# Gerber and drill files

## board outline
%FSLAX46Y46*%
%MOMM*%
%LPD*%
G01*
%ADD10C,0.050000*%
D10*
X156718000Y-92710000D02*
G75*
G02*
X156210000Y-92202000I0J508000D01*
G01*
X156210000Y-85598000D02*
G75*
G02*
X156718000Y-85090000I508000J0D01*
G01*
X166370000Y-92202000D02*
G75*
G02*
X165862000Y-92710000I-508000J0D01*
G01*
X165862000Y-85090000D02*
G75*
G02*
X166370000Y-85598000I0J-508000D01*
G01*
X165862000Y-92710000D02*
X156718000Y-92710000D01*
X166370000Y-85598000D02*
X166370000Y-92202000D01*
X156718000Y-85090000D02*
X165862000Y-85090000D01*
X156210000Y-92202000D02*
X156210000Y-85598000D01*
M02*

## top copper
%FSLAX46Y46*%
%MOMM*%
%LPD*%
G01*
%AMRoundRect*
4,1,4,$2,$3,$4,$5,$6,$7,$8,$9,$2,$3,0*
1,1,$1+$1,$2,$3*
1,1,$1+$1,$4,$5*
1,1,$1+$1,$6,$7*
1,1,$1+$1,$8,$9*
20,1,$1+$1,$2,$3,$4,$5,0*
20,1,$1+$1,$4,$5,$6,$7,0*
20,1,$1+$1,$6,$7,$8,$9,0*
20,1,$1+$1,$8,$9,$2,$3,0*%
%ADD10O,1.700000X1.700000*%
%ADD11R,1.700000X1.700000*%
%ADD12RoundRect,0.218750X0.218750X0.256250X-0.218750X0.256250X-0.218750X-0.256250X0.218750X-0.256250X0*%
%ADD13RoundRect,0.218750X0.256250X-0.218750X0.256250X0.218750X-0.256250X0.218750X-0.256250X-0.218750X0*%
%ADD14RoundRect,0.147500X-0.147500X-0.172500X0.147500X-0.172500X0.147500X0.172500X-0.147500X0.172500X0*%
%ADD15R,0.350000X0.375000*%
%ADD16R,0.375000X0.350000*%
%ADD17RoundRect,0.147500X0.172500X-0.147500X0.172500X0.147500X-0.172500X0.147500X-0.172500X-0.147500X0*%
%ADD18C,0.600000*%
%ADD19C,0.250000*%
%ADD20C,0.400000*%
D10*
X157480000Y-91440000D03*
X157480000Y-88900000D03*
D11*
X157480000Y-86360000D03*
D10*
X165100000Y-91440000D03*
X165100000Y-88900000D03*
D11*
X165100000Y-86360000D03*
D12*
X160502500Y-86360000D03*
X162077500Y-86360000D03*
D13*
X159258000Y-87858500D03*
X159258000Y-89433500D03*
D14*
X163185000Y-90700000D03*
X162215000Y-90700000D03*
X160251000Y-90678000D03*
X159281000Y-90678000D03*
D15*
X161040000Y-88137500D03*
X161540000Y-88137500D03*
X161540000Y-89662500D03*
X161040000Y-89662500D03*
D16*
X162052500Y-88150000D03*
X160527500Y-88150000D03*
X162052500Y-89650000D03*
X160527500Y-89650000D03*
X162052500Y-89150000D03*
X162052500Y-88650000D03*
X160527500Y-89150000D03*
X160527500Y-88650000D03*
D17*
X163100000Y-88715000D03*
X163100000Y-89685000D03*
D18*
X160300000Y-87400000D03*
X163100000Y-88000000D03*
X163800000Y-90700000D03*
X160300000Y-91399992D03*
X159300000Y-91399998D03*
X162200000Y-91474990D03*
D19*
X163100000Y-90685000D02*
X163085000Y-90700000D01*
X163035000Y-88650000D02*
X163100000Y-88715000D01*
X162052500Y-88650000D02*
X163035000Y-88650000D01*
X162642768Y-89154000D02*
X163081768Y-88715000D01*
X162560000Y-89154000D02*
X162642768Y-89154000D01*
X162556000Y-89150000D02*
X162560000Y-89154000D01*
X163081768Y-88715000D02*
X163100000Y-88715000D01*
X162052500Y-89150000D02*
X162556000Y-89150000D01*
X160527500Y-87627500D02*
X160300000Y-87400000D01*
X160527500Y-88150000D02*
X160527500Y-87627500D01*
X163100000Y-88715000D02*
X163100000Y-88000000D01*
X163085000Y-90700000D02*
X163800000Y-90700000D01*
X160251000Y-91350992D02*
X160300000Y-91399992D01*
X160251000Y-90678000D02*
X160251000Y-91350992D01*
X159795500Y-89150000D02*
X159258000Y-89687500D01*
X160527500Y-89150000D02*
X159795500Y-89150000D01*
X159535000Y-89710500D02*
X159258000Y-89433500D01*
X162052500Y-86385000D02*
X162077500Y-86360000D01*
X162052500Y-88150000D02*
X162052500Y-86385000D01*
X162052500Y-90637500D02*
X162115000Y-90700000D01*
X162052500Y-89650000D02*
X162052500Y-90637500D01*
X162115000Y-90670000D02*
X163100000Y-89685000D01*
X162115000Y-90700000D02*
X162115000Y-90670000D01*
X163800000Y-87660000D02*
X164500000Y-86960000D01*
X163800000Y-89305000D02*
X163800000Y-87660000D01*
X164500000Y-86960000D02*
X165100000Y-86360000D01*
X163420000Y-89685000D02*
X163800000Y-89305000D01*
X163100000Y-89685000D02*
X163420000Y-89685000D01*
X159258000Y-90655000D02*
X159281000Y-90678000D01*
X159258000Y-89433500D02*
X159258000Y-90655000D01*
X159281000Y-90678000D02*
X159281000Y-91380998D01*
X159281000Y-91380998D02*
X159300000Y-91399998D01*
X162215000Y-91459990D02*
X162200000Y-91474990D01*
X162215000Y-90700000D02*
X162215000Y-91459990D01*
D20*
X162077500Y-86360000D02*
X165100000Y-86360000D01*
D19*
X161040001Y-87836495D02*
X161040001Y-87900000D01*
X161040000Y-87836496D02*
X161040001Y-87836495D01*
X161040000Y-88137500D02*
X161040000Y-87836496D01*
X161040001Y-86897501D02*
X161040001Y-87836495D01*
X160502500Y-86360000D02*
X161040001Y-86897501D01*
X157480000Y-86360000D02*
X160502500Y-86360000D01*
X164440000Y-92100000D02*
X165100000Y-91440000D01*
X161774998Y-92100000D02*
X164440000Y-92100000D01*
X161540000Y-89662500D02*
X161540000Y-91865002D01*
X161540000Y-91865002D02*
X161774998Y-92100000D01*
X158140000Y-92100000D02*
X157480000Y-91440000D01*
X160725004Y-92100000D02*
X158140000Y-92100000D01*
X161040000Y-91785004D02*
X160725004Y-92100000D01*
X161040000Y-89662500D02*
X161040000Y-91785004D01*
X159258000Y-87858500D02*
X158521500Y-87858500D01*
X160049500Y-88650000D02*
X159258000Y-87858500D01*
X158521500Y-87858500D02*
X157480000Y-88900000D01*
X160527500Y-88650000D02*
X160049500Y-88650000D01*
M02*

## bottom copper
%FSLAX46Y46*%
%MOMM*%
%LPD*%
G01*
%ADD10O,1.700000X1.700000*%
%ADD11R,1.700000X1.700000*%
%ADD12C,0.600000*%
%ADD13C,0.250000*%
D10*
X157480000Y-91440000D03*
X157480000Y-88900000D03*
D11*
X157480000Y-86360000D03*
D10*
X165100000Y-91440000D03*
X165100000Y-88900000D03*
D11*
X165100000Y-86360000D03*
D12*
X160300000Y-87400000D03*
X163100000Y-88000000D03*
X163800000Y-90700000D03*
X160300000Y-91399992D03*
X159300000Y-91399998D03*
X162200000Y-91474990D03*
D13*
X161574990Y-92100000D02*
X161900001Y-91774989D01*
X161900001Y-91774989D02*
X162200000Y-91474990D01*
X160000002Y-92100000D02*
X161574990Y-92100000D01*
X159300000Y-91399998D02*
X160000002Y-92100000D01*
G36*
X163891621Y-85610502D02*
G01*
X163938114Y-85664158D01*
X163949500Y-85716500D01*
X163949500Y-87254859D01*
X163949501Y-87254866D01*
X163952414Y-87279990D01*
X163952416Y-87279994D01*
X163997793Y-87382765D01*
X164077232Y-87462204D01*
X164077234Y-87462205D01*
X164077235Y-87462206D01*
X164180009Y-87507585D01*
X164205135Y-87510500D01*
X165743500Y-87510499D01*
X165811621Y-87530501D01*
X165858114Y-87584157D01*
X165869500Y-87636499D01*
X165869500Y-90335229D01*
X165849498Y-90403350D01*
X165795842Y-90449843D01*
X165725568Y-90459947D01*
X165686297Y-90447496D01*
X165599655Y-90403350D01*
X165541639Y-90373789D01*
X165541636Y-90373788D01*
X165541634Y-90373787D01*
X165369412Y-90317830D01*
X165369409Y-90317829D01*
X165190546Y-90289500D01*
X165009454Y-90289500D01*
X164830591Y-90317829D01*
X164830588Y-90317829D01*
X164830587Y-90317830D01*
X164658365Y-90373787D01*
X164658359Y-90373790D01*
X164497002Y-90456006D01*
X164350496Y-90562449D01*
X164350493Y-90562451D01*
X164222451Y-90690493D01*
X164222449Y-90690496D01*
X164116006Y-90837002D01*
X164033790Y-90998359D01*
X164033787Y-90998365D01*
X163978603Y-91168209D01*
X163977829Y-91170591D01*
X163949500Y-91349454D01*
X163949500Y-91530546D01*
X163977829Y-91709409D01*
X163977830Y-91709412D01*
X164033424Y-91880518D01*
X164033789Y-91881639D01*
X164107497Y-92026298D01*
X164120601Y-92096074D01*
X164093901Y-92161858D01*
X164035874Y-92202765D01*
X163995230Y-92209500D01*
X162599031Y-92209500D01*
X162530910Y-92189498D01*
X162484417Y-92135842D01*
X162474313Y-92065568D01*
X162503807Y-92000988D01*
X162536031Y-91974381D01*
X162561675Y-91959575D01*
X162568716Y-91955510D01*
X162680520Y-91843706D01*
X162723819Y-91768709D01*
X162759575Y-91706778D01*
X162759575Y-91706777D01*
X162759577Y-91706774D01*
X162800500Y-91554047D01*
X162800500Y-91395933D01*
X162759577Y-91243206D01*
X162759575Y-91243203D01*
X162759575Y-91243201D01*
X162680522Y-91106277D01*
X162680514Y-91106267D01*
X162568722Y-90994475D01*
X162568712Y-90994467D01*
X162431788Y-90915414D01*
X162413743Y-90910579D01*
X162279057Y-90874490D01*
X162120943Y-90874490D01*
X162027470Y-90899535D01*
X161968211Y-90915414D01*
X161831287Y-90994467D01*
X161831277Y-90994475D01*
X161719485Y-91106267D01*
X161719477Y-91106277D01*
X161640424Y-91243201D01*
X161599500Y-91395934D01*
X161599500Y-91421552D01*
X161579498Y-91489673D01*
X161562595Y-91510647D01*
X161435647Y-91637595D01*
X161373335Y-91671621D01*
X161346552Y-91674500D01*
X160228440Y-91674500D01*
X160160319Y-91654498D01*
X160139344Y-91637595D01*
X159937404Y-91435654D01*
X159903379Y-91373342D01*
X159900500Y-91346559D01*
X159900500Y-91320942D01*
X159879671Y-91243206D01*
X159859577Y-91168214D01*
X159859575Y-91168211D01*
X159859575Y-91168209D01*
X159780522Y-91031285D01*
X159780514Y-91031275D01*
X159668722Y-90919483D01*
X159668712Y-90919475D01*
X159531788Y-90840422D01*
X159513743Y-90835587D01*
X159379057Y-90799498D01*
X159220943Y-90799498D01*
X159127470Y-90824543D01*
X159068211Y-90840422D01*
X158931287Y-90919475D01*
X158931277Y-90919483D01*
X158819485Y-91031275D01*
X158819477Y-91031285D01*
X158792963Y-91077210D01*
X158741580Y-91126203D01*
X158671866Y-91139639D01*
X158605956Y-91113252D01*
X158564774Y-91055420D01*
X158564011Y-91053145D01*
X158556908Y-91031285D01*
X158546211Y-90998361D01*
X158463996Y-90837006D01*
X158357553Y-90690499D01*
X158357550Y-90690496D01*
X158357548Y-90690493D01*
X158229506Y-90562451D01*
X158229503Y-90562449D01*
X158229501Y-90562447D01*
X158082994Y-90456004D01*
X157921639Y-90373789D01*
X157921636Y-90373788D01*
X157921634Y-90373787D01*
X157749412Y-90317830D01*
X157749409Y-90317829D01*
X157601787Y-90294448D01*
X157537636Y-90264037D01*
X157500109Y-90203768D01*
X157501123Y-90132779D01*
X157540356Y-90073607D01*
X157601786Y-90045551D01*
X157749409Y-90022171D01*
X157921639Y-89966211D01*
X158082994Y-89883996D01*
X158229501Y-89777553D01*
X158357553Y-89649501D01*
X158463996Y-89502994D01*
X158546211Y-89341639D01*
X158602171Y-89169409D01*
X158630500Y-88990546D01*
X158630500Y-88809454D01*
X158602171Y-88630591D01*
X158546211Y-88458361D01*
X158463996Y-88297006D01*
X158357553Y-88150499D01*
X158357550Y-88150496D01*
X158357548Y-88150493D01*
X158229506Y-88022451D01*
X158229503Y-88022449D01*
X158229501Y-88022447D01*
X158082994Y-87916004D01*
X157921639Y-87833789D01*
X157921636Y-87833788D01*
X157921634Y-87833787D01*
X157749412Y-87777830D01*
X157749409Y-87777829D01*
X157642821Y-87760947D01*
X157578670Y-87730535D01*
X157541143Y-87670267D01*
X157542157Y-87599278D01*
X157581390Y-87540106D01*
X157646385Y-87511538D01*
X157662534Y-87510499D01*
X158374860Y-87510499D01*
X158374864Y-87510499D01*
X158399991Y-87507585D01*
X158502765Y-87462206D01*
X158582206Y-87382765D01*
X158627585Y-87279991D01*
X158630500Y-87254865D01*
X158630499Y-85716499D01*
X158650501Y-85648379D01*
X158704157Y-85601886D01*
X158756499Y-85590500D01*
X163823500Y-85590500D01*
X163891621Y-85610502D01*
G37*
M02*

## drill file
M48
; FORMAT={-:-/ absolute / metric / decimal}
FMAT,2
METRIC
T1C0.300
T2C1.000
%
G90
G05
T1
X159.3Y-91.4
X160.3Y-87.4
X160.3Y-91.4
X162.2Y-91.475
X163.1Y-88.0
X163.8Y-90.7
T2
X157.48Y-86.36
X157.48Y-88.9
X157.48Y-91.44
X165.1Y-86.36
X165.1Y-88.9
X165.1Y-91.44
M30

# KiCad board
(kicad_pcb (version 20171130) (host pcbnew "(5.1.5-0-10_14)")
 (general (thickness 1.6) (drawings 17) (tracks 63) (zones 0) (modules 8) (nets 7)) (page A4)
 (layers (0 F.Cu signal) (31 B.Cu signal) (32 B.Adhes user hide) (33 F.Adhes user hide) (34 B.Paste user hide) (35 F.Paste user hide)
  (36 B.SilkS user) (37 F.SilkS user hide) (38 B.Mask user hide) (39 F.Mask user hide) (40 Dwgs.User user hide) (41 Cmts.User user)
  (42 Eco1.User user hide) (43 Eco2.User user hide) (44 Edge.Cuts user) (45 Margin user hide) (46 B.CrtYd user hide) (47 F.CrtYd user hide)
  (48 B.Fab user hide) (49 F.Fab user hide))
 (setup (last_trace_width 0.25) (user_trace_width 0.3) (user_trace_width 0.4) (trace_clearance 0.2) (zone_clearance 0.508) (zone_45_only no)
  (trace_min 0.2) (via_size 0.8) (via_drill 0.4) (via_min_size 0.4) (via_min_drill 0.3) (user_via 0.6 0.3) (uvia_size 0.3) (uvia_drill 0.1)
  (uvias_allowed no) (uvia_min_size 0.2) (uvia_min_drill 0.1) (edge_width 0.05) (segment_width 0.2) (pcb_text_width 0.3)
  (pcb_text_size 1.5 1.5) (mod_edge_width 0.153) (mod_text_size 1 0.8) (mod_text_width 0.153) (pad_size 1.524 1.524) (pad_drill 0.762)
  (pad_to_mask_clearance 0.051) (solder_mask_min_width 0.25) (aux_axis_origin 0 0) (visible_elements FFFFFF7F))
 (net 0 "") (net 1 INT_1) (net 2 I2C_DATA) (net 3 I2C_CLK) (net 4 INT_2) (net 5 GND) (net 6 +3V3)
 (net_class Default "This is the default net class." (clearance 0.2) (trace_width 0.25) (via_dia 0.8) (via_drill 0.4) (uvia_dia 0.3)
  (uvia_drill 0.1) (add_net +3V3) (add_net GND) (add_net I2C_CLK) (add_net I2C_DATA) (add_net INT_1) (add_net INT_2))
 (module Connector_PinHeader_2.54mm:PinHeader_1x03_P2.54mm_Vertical (layer B.Cu) (at 157.48 86.36 180)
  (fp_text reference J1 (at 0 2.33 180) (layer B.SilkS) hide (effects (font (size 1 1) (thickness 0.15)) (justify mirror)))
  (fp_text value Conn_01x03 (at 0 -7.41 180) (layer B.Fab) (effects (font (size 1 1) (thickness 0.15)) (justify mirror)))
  (pad 3 thru_hole oval (at 0 -5.08 180) (size 1.7 1.7) (drill 1) (layers *.Cu *.Mask) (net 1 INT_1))
  (pad 2 thru_hole oval (at 0 -2.54 180) (size 1.7 1.7) (drill 1) (layers *.Cu *.Mask) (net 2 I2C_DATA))
  (pad 1 thru_hole rect (at 0 0 180) (size 1.7 1.7) (drill 1) (layers *.Cu *.Mask) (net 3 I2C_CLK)))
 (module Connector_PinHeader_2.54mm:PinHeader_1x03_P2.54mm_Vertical (layer B.Cu) (at 165.1 86.36 180)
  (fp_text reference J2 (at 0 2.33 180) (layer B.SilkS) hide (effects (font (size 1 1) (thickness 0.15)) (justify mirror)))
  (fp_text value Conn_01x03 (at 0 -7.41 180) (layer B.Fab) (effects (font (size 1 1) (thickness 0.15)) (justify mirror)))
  (pad 3 thru_hole oval (at 0 -5.08 180) (size 1.7 1.7) (drill 1) (layers *.Cu *.Mask) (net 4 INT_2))
  (pad 2 thru_hole oval (at 0 -2.54 180) (size 1.7 1.7) (drill 1) (layers *.Cu *.Mask) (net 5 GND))
  (pad 1 thru_hole rect (at 0 0 180) (size 1.7 1.7) (drill 1) (layers *.Cu *.Mask) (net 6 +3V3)))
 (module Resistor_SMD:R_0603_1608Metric (layer F.Cu) (at 161.29 86.36 180)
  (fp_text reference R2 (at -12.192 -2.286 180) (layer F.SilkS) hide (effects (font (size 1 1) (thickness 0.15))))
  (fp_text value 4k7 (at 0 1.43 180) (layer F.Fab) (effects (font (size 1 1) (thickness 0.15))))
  (pad 2 smd roundrect (at 0.7875 0 180) (size 0.875 0.95) (layers F.Cu F.Paste F.Mask) (roundrect_rratio 0.25) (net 3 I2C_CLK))
  (pad 1 smd roundrect (at -0.7875 0 180) (size 0.875 0.95) (layers F.Cu F.Paste F.Mask) (roundrect_rratio 0.25) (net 6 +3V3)))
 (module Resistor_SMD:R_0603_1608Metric (layer F.Cu) (at 159.258 88.646 90)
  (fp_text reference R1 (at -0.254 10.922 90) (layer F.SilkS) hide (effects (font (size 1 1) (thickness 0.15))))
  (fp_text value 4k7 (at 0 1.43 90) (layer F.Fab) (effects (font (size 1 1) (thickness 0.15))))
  (pad 2 smd roundrect (at 0.7875 0 90) (size 0.875 0.95) (layers F.Cu F.Paste F.Mask) (roundrect_rratio 0.25) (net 2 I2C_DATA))
  (pad 1 smd roundrect (at -0.7875 0 90) (size 0.875 0.95) (layers F.Cu F.Paste F.Mask) (roundrect_rratio 0.25) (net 6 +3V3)))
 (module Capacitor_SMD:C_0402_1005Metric (layer F.Cu) (at 162.7 90.7)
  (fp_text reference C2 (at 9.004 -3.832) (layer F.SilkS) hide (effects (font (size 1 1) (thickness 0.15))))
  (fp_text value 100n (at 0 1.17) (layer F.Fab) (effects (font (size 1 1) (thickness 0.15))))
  (pad 2 smd roundrect (at 0.485 0) (size 0.59 0.64) (layers F.Cu F.Paste F.Mask) (roundrect_rratio 0.25) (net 5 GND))
  (pad 1 smd roundrect (at -0.485 0) (size 0.59 0.64) (layers F.Cu F.Paste F.Mask) (roundrect_rratio 0.25) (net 6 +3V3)))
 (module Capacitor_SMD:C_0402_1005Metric (layer F.Cu) (at 159.766 90.678)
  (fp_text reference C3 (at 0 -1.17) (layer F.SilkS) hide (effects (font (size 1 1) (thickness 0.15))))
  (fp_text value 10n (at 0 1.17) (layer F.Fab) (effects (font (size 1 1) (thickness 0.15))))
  (pad 2 smd roundrect (at 0.485 0) (size 0.59 0.64) (layers F.Cu F.Paste F.Mask) (roundrect_rratio 0.25) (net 5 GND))
  (pad 1 smd roundrect (at -0.485 0) (size 0.59 0.64) (layers F.Cu F.Paste F.Mask) (roundrect_rratio 0.25) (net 6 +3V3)))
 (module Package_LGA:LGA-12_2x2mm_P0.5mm (layer F.Cu) (at 161.29 88.9)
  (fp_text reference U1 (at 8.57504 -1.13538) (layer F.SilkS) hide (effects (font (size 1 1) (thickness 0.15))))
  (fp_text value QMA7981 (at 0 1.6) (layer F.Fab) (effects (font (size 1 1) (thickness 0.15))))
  (pad 12 smd rect (at -0.25 -0.7625 90) (size 0.375 0.35) (layers F.Cu F.Paste F.Mask) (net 3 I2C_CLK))
  (pad 11 smd rect (at 0.25 -0.7625 90) (size 0.375 0.35) (layers F.Cu F.Paste F.Mask))
  (pad 6 smd rect (at 0.25 0.7625 90) (size 0.375 0.35) (layers F.Cu F.Paste F.Mask) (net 4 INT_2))
  (pad 5 smd rect (at -0.25 0.7625 90) (size 0.375 0.35) (layers F.Cu F.Paste F.Mask) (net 1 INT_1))
  (pad 10 smd rect (at 0.7625 -0.75) (size 0.375 0.35) (layers F.Cu F.Paste F.Mask) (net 6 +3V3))
  (pad 1 smd rect (at -0.7625 -0.75) (size 0.375 0.35) (layers F.Cu F.Paste F.Mask) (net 5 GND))
  (pad 7 smd rect (at 0.7625 0.75) (size 0.375 0.35) (layers F.Cu F.Paste F.Mask) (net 6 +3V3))
  (pad 4 smd rect (at -0.7625 0.75) (size 0.375 0.35) (layers F.Cu F.Paste F.Mask))
  (pad 8 smd rect (at 0.7625 0.25) (size 0.375 0.35) (layers F.Cu F.Paste F.Mask) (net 5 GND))
  (pad 9 smd rect (at 0.7625 -0.25) (size 0.375 0.35) (layers F.Cu F.Paste F.Mask) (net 5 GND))
  (pad 3 smd rect (at -0.7625 0.25) (size 0.375 0.35) (layers F.Cu F.Paste F.Mask) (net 6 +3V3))
  (pad 2 smd rect (at -0.7625 -0.25) (size 0.375 0.35) (layers F.Cu F.Paste F.Mask) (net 2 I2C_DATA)))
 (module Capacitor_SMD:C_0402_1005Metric (layer F.Cu) (at 163.1 89.2 90)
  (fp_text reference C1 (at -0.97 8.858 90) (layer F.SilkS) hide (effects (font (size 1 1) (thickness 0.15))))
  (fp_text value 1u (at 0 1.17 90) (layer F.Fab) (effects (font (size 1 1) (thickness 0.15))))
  (pad 2 smd roundrect (at 0.485 0 90) (size 0.59 0.64) (layers F.Cu F.Paste F.Mask) (roundrect_rratio 0.25) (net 5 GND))
  (pad 1 smd roundrect (at -0.485 0 90) (size 0.59 0.64) (layers F.Cu F.Paste F.Mask) (roundrect_rratio 0.25) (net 6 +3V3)))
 (gr_arc (start 156.718 92.202) (end 156.21 92.202) (angle -90) (layer Edge.Cuts) (width 0.05))
 (gr_arc (start 156.718 85.598) (end 156.718 85.09) (angle -90) (layer Edge.Cuts) (width 0.05))
 (gr_arc (start 165.862 92.202) (end 165.862 92.71) (angle -90) (layer Edge.Cuts) (width 0.05))
 (gr_arc (start 165.862 85.598) (end 166.37 85.598) (angle -90) (layer Edge.Cuts) (width 0.05))
 (gr_line (start 165.862 92.71) (end 156.718 92.71) (layer Edge.Cuts) (width 0.05))
 (gr_line (start 166.37 85.598) (end 166.37 92.202) (layer Edge.Cuts) (width 0.05))
 (gr_line (start 156.718 85.09) (end 165.862 85.09) (layer Edge.Cuts) (width 0.05))
 (gr_line (start 156.21 92.202) (end 156.21 85.598) (layer Edge.Cuts) (width 0.05))
 (segment (start 163.1 90.685) (end 163.085 90.7) (width 0.25) (layer F.Cu) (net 5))
 (segment (start 163.035 88.65) (end 163.1 88.715) (width 0.25) (layer F.Cu) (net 5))
 (segment (start 162.0525 88.65) (end 163.035 88.65) (width 0.25) (layer F.Cu) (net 5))
 (segment (start 162.642768 89.154) (end 163.081768 88.715) (width 0.25) (layer F.Cu) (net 5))
 (segment (start 162.56 89.154) (end 162.642768 89.154) (width 0.25) (layer F.Cu) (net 5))
 (segment (start 162.556 89.15) (end 162.56 89.154) (width 0.25) (layer F.Cu) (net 5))
 (segment (start 163.081768 88.715) (end 163.1 88.715) (width 0.25) (layer F.Cu) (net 5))
 (segment (start 162.0525 89.15) (end 162.556 89.15) (width 0.25) (layer F.Cu) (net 5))
 (via (at 160.3 87.4) (size 0.6) (drill 0.3) (layers F.Cu B.Cu) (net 5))
 (segment (start 160.5275 87.6275) (end 160.3 87.4) (width 0.25) (layer F.Cu) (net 5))
 (segment (start 160.5275 88.15) (end 160.5275 87.6275) (width 0.25) (layer F.Cu) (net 5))
 (via (at 163.1 88) (size 0.6) (drill 0.3) (layers F.Cu B.Cu) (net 5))
 (segment (start 163.1 88.715) (end 163.1 88) (width 0.25) (layer F.Cu) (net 5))
 (segment (start 163.085 90.7) (end 163.8 90.7) (width 0.25) (layer F.Cu) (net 5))
 (via (at 163.8 90.7) (size 0.6) (drill 0.3) (layers F.Cu B.Cu) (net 5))
 (via (at 160.3 91.399992) (size 0.6) (drill 0.3) (layers F.Cu B.Cu) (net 5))
 (segment (start 160.251 91.350992) (end 160.3 91.399992) (width 0.25) (layer F.Cu) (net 5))
 (segment (start 160.251 90.678) (end 160.251 91.350992) (width 0.25) (layer F.Cu) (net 5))
 (segment (start 159.7955 89.15) (end 159.258 89.6875) (width 0.25) (layer F.Cu) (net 6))
 (segment (start 160.5275 89.15) (end 159.7955 89.15) (width 0.25) (layer F.Cu) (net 6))
 (segment (start 159.535 89.7105) (end 159.258 89.4335) (width 0.25) (layer F.Cu) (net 6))
 (segment (start 162.0525 86.385) (end 162.0775 86.36) (width 0.25) (layer F.Cu) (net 6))
 (segment (start 162.0525 88.15) (end 162.0525 86.385) (width 0.25) (layer F.Cu) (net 6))
 (segment (start 162.0525 90.6375) (end 162.115 90.7) (width 0.25) (layer F.Cu) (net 6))
 (segment (start 162.0525 89.65) (end 162.0525 90.6375) (width 0.25) (layer F.Cu) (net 6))
 (segment (start 162.115 90.67) (end 163.1 89.685) (width 0.25) (layer F.Cu) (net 6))
 (segment (start 162.115 90.7) (end 162.115 90.67) (width 0.25) (layer F.Cu) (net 6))
 (segment (start 163.8 87.66) (end 164.5 86.96) (width 0.25) (layer F.Cu) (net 6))
 (segment (start 163.8 89.305) (end 163.8 87.66) (width 0.25) (layer F.Cu) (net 6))
 (segment (start 164.5 86.96) (end 165.1 86.36) (width 0.25) (layer F.Cu) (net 6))
 (segment (start 163.42 89.685) (end 163.8 89.305) (width 0.25) (layer F.Cu) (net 6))
 (segment (start 163.1 89.685) (end 163.42 89.685) (width 0.25) (layer F.Cu) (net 6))
 (segment (start 159.258 90.655) (end 159.281 90.678) (width 0.25) (layer F.Cu) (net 6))
 (segment (start 159.258 89.4335) (end 159.258 90.655) (width 0.25) (layer F.Cu) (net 6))
 (via (at 159.3 91.399998) (size 0.6) (drill 0.3) (layers F.Cu B.Cu) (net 6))
 (segment (start 159.281 90.678) (end 159.281 91.380998) (width 0.25) (layer F.Cu) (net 6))
 (segment (start 159.281 91.380998) (end 159.3 91.399998) (width 0.25) (layer F.Cu) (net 6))
 (via (at 162.2 91.47499) (size 0.6) (drill 0.3) (layers F.Cu B.Cu) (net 6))
 (segment (start 161.57499 92.1) (end 161.900001 91.774989) (width 0.25) (layer B.Cu) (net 6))
 (segment (start 162.215 91.45999) (end 162.2 91.47499) (width 0.25) (layer F.Cu) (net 6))
 (segment (start 161.900001 91.774989) (end 162.2 91.47499) (width 0.25) (layer B.Cu) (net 6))
 (segment (start 160.000002 92.1) (end 161.57499 92.1) (width 0.25) (layer B.Cu) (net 6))
 (segment (start 162.215 90.7) (end 162.215 91.45999) (width 0.25) (layer F.Cu) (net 6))
 (segment (start 159.3 91.399998) (end 160.000002 92.1) (width 0.25) (layer B.Cu) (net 6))
 (segment (start 162.0775 86.36) (end 165.1 86.36) (width 0.4) (layer F.Cu) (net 6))
 (segment (start 161.040001 87.836495) (end 161.040001 87.9) (width 0.25) (layer F.Cu) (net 3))
 (segment (start 161.04 87.836496) (end 161.040001 87.836495) (width 0.25) (layer F.Cu) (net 3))
 (segment (start 161.04 88.1375) (end 161.04 87.836496) (width 0.25) (layer F.Cu) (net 3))
 (segment (start 161.040001 86.897501) (end 161.040001 87.836495) (width 0.25) (layer F.Cu) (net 3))
 (segment (start 160.5025 86.36) (end 161.040001 86.897501) (width 0.25) (layer F.Cu) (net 3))
 (segment (start 157.48 86.36) (end 160.5025 86.36) (width 0.25) (layer F.Cu) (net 3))
 (segment (start 164.44 92.1) (end 165.1 91.44) (width 0.25) (layer F.Cu) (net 4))
 (segment (start 161.774998 92.1) (end 164.44 92.1) (width 0.25) (layer F.Cu) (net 4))
 (segment (start 161.54 89.6625) (end 161.54 91.865002) (width 0.25) (layer F.Cu) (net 4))
 (segment (start 161.54 91.865002) (end 161.774998 92.1) (width 0.25) (layer F.Cu) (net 4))
 (segment (start 158.14 92.1) (end 157.48 91.44) (width 0.25) (layer F.Cu) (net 1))
 (segment (start 160.725004 92.1) (end 158.14 92.1) (width 0.25) (layer F.Cu) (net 1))
 (segment (start 161.04 91.785004) (end 160.725004 92.1) (width 0.25) (layer F.Cu) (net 1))
 (segment (start 161.04 89.6625) (end 161.04 91.785004) (width 0.25) (layer F.Cu) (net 1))
 (segment (start 159.258 87.8585) (end 158.5215 87.8585) (width 0.25) (layer F.Cu) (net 2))
 (segment (start 160.0495 88.65) (end 159.258 87.8585) (width 0.25) (layer F.Cu) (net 2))
 (segment (start 158.5215 87.8585) (end 157.48 88.9) (width 0.25) (layer F.Cu) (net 2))
 (segment (start 160.5275 88.65) (end 160.0495 88.65) (width 0.25) (layer F.Cu) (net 2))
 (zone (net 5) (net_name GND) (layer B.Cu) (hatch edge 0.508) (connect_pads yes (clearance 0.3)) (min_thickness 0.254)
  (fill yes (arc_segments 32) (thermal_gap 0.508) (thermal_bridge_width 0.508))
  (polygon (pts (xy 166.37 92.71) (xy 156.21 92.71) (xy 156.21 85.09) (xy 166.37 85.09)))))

